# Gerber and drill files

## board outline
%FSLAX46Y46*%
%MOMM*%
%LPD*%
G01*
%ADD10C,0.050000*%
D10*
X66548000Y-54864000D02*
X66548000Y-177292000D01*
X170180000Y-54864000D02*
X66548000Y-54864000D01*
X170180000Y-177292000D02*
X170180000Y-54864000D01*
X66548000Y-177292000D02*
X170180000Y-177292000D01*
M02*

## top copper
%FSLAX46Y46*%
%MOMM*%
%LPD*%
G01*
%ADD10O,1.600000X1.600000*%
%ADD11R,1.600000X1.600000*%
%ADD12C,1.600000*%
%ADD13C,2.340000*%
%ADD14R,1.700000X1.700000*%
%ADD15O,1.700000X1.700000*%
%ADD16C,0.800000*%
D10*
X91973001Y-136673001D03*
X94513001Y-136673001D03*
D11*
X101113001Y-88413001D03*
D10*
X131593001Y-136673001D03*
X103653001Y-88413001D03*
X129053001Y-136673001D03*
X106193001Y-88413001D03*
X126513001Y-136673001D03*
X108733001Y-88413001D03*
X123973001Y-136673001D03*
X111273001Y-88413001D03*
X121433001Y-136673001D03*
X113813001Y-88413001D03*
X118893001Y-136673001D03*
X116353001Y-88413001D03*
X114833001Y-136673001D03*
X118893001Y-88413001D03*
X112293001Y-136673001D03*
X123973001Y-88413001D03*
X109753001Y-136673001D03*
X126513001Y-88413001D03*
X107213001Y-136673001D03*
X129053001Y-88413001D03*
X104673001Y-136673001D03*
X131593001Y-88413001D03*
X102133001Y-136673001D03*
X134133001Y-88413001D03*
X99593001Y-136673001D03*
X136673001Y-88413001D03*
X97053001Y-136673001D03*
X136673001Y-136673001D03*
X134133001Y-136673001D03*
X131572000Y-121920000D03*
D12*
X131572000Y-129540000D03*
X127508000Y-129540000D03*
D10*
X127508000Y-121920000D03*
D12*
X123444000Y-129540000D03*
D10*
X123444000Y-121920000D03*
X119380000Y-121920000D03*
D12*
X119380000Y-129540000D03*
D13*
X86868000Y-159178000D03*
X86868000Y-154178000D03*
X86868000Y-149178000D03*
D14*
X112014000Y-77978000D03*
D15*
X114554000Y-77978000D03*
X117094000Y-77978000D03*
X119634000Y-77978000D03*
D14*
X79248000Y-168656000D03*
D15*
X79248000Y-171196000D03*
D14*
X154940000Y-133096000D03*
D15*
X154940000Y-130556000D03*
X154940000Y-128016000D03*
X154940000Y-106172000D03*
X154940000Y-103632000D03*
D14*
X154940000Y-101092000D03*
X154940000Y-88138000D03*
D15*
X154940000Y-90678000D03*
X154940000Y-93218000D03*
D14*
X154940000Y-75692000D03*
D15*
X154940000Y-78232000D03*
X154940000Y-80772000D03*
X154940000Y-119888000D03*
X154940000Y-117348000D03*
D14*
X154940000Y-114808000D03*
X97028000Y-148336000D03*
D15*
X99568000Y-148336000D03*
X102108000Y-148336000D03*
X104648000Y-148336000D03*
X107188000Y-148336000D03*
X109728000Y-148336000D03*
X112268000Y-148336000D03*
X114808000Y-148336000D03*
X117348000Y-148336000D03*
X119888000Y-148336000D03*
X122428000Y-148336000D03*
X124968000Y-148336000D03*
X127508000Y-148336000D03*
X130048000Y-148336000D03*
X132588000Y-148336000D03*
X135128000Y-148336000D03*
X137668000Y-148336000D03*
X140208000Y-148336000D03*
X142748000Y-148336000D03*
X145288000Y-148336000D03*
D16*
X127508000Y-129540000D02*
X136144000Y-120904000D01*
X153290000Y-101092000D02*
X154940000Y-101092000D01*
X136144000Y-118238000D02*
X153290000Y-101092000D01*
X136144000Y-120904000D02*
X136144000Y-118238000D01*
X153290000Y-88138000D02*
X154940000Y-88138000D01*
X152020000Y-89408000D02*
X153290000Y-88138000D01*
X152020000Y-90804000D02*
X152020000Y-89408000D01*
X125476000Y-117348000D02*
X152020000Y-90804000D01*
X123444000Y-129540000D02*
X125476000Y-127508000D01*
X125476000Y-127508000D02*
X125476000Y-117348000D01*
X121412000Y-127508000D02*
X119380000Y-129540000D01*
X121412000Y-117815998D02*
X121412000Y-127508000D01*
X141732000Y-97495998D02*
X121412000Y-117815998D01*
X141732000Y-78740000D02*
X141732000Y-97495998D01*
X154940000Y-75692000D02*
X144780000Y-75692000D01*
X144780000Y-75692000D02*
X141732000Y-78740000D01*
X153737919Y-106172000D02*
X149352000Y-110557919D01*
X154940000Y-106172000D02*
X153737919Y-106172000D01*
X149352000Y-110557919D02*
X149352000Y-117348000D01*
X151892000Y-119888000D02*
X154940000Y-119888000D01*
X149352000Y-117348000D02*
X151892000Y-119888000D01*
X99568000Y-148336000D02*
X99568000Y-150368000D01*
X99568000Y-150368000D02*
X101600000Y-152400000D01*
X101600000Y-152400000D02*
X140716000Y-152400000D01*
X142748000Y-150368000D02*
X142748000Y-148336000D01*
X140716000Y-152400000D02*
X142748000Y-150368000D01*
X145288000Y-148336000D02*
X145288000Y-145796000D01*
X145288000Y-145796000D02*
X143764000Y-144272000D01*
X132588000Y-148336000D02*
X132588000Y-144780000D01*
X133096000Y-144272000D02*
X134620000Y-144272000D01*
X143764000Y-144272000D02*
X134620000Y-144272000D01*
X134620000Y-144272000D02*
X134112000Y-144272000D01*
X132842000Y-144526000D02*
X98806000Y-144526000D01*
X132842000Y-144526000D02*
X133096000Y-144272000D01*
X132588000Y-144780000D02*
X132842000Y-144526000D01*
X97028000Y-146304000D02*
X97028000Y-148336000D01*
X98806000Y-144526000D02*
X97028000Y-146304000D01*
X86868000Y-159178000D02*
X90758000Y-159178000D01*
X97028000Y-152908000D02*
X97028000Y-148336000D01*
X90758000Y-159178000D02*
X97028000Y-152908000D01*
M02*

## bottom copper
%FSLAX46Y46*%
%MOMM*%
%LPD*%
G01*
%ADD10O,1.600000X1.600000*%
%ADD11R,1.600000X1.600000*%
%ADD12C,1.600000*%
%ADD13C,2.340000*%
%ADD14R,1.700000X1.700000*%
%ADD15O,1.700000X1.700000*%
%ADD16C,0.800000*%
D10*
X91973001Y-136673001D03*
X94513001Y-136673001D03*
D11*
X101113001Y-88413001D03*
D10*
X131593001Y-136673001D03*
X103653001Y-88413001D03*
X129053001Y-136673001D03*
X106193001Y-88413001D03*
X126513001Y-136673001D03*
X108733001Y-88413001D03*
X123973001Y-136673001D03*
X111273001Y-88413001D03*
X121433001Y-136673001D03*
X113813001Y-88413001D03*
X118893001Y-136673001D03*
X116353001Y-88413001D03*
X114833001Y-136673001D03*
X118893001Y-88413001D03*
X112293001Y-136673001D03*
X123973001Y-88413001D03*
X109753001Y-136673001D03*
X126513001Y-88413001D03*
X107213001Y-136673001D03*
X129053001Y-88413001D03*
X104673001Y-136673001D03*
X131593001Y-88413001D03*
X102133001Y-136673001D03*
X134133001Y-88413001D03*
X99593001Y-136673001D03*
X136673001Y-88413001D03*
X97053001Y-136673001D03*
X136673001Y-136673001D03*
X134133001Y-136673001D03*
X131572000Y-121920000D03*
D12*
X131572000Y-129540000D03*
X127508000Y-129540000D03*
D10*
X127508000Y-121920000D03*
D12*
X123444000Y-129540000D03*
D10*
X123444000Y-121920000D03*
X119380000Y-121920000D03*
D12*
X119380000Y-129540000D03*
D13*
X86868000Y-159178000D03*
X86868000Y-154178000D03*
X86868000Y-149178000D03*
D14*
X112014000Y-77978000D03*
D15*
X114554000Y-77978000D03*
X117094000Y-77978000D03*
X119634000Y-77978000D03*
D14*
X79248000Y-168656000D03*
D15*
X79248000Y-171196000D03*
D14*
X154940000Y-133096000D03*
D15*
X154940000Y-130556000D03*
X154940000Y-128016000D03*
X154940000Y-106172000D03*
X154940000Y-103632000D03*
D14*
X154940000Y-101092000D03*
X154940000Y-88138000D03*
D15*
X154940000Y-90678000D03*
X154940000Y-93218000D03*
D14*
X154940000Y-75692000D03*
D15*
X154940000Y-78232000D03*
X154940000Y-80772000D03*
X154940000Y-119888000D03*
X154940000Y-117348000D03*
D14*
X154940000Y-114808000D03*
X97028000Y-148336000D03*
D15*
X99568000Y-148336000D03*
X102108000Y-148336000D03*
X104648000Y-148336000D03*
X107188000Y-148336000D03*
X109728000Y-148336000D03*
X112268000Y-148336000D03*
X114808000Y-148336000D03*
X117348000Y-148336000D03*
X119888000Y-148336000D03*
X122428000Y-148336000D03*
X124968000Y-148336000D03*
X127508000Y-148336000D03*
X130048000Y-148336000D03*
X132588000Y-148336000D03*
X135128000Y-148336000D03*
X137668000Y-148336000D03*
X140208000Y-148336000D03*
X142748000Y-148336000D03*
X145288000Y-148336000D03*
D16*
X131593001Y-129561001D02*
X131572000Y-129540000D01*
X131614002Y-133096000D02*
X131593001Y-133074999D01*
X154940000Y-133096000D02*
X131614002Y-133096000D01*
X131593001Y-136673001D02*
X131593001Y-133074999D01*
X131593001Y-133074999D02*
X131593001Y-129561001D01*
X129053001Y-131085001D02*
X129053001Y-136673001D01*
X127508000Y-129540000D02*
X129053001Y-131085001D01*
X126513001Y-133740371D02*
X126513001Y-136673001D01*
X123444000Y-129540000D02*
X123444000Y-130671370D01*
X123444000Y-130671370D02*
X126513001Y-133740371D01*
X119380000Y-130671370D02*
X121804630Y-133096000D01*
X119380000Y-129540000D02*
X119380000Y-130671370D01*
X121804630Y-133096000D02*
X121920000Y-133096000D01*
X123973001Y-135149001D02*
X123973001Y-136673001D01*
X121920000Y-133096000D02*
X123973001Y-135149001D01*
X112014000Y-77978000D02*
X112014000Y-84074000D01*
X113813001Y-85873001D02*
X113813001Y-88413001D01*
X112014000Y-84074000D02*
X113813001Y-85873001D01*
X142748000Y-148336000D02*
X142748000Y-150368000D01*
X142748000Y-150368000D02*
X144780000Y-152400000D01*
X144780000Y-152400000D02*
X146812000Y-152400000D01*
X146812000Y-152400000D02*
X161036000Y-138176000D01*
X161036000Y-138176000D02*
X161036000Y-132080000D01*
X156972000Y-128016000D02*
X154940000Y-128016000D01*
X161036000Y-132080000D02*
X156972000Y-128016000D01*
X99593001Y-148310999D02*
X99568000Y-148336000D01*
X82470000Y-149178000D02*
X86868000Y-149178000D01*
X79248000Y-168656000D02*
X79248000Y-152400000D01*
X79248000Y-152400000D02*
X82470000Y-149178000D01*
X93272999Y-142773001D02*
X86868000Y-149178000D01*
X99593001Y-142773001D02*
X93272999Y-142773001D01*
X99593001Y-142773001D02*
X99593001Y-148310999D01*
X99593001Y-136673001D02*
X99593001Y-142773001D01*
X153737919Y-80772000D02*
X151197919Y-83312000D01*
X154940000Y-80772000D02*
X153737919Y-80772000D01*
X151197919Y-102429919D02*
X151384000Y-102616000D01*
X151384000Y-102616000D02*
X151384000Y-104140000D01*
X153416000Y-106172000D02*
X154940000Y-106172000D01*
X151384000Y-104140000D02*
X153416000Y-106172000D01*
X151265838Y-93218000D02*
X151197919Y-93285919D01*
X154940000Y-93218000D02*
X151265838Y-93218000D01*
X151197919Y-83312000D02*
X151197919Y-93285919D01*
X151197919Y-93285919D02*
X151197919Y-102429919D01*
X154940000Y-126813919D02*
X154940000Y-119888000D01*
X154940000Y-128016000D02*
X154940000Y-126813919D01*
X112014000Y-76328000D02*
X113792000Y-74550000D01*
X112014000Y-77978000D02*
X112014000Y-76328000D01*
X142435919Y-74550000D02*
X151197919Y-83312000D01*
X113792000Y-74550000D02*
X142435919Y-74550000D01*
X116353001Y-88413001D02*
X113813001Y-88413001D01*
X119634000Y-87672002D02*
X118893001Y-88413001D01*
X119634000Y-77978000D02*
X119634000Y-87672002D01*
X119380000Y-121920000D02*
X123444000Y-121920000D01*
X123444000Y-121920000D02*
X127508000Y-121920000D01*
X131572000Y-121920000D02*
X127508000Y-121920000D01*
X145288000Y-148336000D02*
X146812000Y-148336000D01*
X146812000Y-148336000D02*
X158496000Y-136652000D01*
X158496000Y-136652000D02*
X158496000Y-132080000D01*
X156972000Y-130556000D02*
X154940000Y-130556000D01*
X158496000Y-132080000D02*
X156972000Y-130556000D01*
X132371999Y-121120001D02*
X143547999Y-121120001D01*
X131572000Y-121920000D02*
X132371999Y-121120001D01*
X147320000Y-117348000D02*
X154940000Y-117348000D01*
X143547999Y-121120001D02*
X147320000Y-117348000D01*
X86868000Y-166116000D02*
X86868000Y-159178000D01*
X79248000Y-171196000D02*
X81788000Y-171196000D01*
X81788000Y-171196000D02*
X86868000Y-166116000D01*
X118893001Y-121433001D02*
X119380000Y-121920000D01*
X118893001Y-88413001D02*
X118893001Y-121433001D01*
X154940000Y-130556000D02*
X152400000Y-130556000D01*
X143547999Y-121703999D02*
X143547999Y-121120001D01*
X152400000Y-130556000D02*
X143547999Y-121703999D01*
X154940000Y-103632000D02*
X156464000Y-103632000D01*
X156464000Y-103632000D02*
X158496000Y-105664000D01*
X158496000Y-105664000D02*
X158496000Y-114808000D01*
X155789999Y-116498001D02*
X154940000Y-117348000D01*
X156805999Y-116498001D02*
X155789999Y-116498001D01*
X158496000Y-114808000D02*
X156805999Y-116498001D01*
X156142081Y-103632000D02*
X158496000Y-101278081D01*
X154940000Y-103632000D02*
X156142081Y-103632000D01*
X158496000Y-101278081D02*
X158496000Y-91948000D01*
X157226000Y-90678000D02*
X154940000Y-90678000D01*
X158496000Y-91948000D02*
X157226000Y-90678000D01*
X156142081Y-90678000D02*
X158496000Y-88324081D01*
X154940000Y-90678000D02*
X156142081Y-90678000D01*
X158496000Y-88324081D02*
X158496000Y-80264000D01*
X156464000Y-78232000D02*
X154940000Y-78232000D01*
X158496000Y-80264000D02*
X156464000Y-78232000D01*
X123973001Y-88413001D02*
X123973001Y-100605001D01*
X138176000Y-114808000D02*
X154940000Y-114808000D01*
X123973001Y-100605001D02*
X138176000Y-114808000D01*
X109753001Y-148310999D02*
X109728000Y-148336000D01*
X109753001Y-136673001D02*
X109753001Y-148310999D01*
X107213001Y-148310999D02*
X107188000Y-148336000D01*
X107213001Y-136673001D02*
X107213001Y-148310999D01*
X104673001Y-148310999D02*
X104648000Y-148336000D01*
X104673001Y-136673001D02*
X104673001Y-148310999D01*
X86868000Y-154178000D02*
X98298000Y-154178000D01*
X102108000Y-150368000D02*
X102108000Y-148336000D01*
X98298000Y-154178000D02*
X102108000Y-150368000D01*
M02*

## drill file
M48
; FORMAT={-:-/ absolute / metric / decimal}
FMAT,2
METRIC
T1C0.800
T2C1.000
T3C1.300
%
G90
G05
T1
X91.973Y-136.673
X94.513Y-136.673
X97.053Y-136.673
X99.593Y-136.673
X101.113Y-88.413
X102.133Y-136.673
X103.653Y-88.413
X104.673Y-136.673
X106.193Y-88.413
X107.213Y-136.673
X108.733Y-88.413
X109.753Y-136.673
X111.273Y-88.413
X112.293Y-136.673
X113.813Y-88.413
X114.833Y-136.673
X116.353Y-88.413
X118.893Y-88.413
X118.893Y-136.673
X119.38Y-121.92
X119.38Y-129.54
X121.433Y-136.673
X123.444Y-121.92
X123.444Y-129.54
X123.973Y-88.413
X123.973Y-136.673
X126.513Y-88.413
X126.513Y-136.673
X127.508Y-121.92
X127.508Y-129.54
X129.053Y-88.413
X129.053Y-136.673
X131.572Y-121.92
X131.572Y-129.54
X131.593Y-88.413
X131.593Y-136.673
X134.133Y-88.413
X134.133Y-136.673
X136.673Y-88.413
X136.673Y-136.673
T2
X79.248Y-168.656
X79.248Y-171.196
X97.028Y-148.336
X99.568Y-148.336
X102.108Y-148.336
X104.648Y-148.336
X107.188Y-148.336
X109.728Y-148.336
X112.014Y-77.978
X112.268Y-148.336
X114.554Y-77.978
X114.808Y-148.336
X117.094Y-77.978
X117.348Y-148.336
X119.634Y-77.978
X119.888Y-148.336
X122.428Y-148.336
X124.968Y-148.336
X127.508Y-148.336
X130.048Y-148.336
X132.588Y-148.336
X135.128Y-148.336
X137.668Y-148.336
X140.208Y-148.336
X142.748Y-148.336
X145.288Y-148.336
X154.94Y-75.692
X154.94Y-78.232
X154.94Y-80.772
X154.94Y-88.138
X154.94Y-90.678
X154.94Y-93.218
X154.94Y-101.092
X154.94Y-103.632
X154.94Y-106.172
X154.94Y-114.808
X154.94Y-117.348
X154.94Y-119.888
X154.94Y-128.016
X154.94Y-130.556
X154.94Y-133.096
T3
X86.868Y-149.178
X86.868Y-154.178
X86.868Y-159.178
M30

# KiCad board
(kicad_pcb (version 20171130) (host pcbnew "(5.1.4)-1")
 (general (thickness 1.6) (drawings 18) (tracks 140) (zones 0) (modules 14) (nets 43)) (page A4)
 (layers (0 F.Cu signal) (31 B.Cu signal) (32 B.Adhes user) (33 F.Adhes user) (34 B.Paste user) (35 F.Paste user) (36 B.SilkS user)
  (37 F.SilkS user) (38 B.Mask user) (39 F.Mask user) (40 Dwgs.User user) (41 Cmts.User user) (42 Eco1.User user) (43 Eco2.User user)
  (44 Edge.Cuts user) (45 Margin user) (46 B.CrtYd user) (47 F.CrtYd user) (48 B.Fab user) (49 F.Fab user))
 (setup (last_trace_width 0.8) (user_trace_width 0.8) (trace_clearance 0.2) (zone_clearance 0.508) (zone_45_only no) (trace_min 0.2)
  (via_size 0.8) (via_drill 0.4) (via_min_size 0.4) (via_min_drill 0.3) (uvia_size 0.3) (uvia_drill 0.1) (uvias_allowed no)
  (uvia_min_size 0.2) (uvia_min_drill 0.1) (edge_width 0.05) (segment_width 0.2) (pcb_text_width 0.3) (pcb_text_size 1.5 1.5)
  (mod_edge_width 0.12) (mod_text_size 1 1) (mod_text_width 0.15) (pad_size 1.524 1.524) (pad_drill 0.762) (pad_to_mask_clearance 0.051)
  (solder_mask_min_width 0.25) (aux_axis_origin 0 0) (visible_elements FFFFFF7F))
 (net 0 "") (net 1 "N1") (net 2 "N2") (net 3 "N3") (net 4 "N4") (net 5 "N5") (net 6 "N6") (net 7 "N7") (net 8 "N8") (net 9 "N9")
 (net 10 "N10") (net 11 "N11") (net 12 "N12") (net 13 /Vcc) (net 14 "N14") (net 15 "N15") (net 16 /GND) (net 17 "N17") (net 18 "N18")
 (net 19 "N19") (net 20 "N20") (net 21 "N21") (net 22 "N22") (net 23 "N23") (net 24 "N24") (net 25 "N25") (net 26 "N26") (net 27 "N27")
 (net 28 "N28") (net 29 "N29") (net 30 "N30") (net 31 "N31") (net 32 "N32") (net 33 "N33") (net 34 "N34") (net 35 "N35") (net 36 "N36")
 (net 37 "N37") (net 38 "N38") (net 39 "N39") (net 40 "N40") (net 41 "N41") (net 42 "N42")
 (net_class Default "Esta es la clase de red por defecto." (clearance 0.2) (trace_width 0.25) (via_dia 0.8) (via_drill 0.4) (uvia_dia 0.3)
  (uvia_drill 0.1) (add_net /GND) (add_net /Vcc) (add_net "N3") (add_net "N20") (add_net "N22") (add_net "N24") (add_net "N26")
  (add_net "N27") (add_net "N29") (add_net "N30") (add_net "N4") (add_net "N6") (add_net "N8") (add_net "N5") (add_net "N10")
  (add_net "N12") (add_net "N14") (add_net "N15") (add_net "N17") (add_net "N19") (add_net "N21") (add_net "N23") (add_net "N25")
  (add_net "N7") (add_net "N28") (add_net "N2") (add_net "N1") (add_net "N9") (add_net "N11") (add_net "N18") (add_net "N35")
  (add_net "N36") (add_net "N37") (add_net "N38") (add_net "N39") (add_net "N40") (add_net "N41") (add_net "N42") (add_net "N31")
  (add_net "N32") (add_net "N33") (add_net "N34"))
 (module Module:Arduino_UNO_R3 (layer F.Cu) (at 101.113001 88.413001)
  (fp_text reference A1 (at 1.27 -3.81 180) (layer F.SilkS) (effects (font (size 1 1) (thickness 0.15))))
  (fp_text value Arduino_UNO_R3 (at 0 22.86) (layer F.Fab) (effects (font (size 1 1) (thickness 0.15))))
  (pad 32 thru_hole oval (at -9.14 48.26 90) (size 1.6 1.6) (drill 0.8) (layers *.Cu *.Mask) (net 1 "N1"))
  (pad 31 thru_hole oval (at -6.6 48.26 90) (size 1.6 1.6) (drill 0.8) (layers *.Cu *.Mask) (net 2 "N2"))
  (pad 1 thru_hole rect (at 0 0 90) (size 1.6 1.6) (drill 0.8) (layers *.Cu *.Mask) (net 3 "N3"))
  (pad 17 thru_hole oval (at 30.48 48.26 90) (size 1.6 1.6) (drill 0.8) (layers *.Cu *.Mask) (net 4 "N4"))
  (pad 2 thru_hole oval (at 2.54 0 90) (size 1.6 1.6) (drill 0.8) (layers *.Cu *.Mask) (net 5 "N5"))
  (pad 18 thru_hole oval (at 27.94 48.26 90) (size 1.6 1.6) (drill 0.8) (layers *.Cu *.Mask) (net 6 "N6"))
  (pad 3 thru_hole oval (at 5.08 0 90) (size 1.6 1.6) (drill 0.8) (layers *.Cu *.Mask) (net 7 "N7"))
  (pad 19 thru_hole oval (at 25.4 48.26 90) (size 1.6 1.6) (drill 0.8) (layers *.Cu *.Mask) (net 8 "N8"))
  (pad 4 thru_hole oval (at 7.62 0 90) (size 1.6 1.6) (drill 0.8) (layers *.Cu *.Mask) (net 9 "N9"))
  (pad 20 thru_hole oval (at 22.86 48.26 90) (size 1.6 1.6) (drill 0.8) (layers *.Cu *.Mask) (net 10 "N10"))
  (pad 5 thru_hole oval (at 10.16 0 90) (size 1.6 1.6) (drill 0.8) (layers *.Cu *.Mask) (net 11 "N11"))
  (pad 21 thru_hole oval (at 20.32 48.26 90) (size 1.6 1.6) (drill 0.8) (layers *.Cu *.Mask) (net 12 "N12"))
  (pad 6 thru_hole oval (at 12.7 0 90) (size 1.6 1.6) (drill 0.8) (layers *.Cu *.Mask) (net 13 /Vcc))
  (pad 22 thru_hole oval (at 17.78 48.26 90) (size 1.6 1.6) (drill 0.8) (layers *.Cu *.Mask) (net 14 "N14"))
  (pad 7 thru_hole oval (at 15.24 0 90) (size 1.6 1.6) (drill 0.8) (layers *.Cu *.Mask) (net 13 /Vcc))
  (pad 23 thru_hole oval (at 13.72 48.26 90) (size 1.6 1.6) (drill 0.8) (layers *.Cu *.Mask) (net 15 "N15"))
  (pad 8 thru_hole oval (at 17.78 0 90) (size 1.6 1.6) (drill 0.8) (layers *.Cu *.Mask) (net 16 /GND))
  (pad 24 thru_hole oval (at 11.18 48.26 90) (size 1.6 1.6) (drill 0.8) (layers *.Cu *.Mask) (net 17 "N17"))
  (pad 9 thru_hole oval (at 22.86 0 90) (size 1.6 1.6) (drill 0.8) (layers *.Cu *.Mask) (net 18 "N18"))
  (pad 25 thru_hole oval (at 8.64 48.26 90) (size 1.6 1.6) (drill 0.8) (layers *.Cu *.Mask) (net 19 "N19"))
  (pad 10 thru_hole oval (at 25.4 0 90) (size 1.6 1.6) (drill 0.8) (layers *.Cu *.Mask) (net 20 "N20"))
  (pad 26 thru_hole oval (at 6.1 48.26 90) (size 1.6 1.6) (drill 0.8) (layers *.Cu *.Mask) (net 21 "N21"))
  (pad 11 thru_hole oval (at 27.94 0 90) (size 1.6 1.6) (drill 0.8) (layers *.Cu *.Mask) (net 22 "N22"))
  (pad 27 thru_hole oval (at 3.56 48.26 90) (size 1.6 1.6) (drill 0.8) (layers *.Cu *.Mask) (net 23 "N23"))
  (pad 12 thru_hole oval (at 30.48 0 90) (size 1.6 1.6) (drill 0.8) (layers *.Cu *.Mask) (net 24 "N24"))
  (pad 28 thru_hole oval (at 1.02 48.26 90) (size 1.6 1.6) (drill 0.8) (layers *.Cu *.Mask) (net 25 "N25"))
  (pad 13 thru_hole oval (at 33.02 0 90) (size 1.6 1.6) (drill 0.8) (layers *.Cu *.Mask) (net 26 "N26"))
  (pad 29 thru_hole oval (at -1.52 48.26 90) (size 1.6 1.6) (drill 0.8) (layers *.Cu *.Mask) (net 13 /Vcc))
  (pad 14 thru_hole oval (at 35.56 0 90) (size 1.6 1.6) (drill 0.8) (layers *.Cu *.Mask) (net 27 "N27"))
  (pad 30 thru_hole oval (at -4.06 48.26 90) (size 1.6 1.6) (drill 0.8) (layers *.Cu *.Mask) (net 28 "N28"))
  (pad 15 thru_hole oval (at 35.56 48.26 90) (size 1.6 1.6) (drill 0.8) (layers *.Cu *.Mask) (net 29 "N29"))
  (pad 16 thru_hole oval (at 33.02 48.26 90) (size 1.6 1.6) (drill 0.8) (layers *.Cu *.Mask) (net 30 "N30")))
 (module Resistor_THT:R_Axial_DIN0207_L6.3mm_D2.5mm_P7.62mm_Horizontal (layer F.Cu) (at 131.572 129.54 90)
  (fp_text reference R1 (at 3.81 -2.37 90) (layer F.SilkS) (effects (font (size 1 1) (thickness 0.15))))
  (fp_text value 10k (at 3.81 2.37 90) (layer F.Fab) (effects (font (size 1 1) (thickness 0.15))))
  (pad 2 thru_hole oval (at 7.62 0 90) (size 1.6 1.6) (drill 0.8) (layers *.Cu *.Mask) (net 16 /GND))
  (pad 1 thru_hole circle (at 0 0 90) (size 1.6 1.6) (drill 0.8) (layers *.Cu *.Mask) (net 4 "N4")))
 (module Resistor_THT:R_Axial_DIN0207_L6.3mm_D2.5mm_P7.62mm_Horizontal (layer F.Cu) (at 127.508 129.54 90)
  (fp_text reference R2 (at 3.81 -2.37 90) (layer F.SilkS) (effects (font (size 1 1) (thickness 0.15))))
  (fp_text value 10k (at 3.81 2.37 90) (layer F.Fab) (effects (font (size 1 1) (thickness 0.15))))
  (pad 1 thru_hole circle (at 0 0 90) (size 1.6 1.6) (drill 0.8) (layers *.Cu *.Mask) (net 6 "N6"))
  (pad 2 thru_hole oval (at 7.62 0 90) (size 1.6 1.6) (drill 0.8) (layers *.Cu *.Mask) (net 16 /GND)))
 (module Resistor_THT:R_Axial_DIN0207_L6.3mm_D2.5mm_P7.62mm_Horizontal (layer F.Cu) (at 123.444 129.54 90)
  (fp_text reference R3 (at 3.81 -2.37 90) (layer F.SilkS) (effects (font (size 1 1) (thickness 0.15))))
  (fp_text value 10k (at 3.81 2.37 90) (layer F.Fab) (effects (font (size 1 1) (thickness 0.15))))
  (pad 1 thru_hole circle (at 0 0 90) (size 1.6 1.6) (drill 0.8) (layers *.Cu *.Mask) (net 8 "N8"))
  (pad 2 thru_hole oval (at 7.62 0 90) (size 1.6 1.6) (drill 0.8) (layers *.Cu *.Mask) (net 16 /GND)))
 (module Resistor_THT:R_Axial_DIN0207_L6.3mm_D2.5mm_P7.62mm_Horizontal (layer F.Cu) (at 119.38 129.54 90)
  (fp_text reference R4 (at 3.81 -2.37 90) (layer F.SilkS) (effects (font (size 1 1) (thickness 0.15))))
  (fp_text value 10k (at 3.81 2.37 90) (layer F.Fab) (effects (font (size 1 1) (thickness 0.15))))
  (pad 2 thru_hole oval (at 7.62 0 90) (size 1.6 1.6) (drill 0.8) (layers *.Cu *.Mask) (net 16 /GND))
  (pad 1 thru_hole circle (at 0 0 90) (size 1.6 1.6) (drill 0.8) (layers *.Cu *.Mask) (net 10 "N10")))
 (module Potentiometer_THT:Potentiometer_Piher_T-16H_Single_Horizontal (layer F.Cu) (at 86.868 149.178 180)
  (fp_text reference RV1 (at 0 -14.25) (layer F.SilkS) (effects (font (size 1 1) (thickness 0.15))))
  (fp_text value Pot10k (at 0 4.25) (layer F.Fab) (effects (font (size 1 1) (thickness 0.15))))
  (pad 3 thru_hole circle (at 0 -10 180) (size 2.34 2.34) (drill 1.3) (layers *.Cu *.Mask) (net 16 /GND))
  (pad 2 thru_hole circle (at 0 -5 180) (size 2.34 2.34) (drill 1.3) (layers *.Cu *.Mask) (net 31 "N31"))
  (pad 1 thru_hole circle (at 0 0 180) (size 2.34 2.34) (drill 1.3) (layers *.Cu *.Mask) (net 13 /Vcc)))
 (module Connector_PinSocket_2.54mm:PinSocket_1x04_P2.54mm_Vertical (layer F.Cu) (at 112.014 77.978 90)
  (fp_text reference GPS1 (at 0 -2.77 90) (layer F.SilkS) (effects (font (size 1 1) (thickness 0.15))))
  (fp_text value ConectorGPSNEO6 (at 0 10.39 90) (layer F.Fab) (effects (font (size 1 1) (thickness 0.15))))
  (pad 1 thru_hole rect (at 0 0 90) (size 1.7 1.7) (drill 1) (layers *.Cu *.Mask) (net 13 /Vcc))
  (pad 2 thru_hole oval (at 0 2.54 90) (size 1.7 1.7) (drill 1) (layers *.Cu *.Mask))
  (pad 3 thru_hole oval (at 0 5.08 90) (size 1.7 1.7) (drill 1) (layers *.Cu *.Mask))
  (pad 4 thru_hole oval (at 0 7.62 90) (size 1.7 1.7) (drill 1) (layers *.Cu *.Mask) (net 16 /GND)))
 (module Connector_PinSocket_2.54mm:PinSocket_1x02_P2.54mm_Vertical (layer F.Cu) (at 79.248 168.656)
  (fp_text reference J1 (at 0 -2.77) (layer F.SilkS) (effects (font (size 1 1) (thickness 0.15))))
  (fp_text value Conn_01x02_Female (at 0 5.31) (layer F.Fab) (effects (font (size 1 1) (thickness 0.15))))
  (pad 1 thru_hole rect (at 0 0) (size 1.7 1.7) (drill 1) (layers *.Cu *.Mask) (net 13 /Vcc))
  (pad 2 thru_hole oval (at 0 2.54) (size 1.7 1.7) (drill 1) (layers *.Cu *.Mask) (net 16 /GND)))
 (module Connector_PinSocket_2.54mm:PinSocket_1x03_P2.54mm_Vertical (layer F.Cu) (at 154.94 133.096 180)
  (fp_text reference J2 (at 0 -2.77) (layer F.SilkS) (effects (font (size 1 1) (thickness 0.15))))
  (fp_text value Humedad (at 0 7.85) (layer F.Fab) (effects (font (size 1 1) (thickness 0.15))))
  (pad 1 thru_hole rect (at 0 0 180) (size 1.7 1.7) (drill 1) (layers *.Cu *.Mask) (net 4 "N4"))
  (pad 2 thru_hole oval (at 0 2.54 180) (size 1.7 1.7) (drill 1) (layers *.Cu *.Mask) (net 16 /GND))
  (pad 3 thru_hole oval (at 0 5.08 180) (size 1.7 1.7) (drill 1) (layers *.Cu *.Mask) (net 13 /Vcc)))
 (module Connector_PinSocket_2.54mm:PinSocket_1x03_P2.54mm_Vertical (layer F.Cu) (at 154.94 101.092)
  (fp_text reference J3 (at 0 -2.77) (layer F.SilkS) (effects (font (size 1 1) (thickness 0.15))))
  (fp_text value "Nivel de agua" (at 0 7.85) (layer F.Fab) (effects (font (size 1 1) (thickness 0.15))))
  (pad 3 thru_hole oval (at 0 5.08) (size 1.7 1.7) (drill 1) (layers *.Cu *.Mask) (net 13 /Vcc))
  (pad 2 thru_hole oval (at 0 2.54) (size 1.7 1.7) (drill 1) (layers *.Cu *.Mask) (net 16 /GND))
  (pad 1 thru_hole rect (at 0 0) (size 1.7 1.7) (drill 1) (layers *.Cu *.Mask) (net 6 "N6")))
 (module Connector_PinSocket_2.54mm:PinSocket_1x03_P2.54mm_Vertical (layer F.Cu) (at 154.94 88.138)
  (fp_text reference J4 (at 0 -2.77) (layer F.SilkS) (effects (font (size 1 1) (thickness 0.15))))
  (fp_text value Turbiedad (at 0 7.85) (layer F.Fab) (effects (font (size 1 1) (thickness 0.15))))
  (pad 1 thru_hole rect (at 0 0) (size 1.7 1.7) (drill 1) (layers *.Cu *.Mask) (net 8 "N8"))
  (pad 2 thru_hole oval (at 0 2.54) (size 1.7 1.7) (drill 1) (layers *.Cu *.Mask) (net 16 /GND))
  (pad 3 thru_hole oval (at 0 5.08) (size 1.7 1.7) (drill 1) (layers *.Cu *.Mask) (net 13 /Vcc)))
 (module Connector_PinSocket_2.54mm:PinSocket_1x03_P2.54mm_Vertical (layer F.Cu) (at 154.94 75.692)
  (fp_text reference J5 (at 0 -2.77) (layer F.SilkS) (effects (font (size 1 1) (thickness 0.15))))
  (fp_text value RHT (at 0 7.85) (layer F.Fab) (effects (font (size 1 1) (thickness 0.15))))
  (pad 1 thru_hole rect (at 0 0) (size 1.7 1.7) (drill 1) (layers *.Cu *.Mask) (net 10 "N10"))
  (pad 2 thru_hole oval (at 0 2.54) (size 1.7 1.7) (drill 1) (layers *.Cu *.Mask) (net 16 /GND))
  (pad 3 thru_hole oval (at 0 5.08) (size 1.7 1.7) (drill 1) (layers *.Cu *.Mask) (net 13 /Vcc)))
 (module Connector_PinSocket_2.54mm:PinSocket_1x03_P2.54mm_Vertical (layer F.Cu) (at 154.94 114.808)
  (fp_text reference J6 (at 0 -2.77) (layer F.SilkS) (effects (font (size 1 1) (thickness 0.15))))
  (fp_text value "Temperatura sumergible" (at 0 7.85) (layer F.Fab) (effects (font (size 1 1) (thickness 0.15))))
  (pad 3 thru_hole oval (at 0 5.08) (size 1.7 1.7) (drill 1) (layers *.Cu *.Mask) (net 13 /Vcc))
  (pad 2 thru_hole oval (at 0 2.54) (size 1.7 1.7) (drill 1) (layers *.Cu *.Mask) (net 16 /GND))
  (pad 1 thru_hole rect (at 0 0) (size 1.7 1.7) (drill 1) (layers *.Cu *.Mask) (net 18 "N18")))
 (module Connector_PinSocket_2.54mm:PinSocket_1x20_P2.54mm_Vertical (layer F.Cu) (at 97.028 148.336 90)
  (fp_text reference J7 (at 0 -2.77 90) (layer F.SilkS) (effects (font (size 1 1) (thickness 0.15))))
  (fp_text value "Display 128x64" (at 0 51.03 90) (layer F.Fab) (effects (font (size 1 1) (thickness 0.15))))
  (pad 1 thru_hole rect (at 0 0 90) (size 1.7 1.7) (drill 1) (layers *.Cu *.Mask) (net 16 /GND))
  (pad 2 thru_hole oval (at 0 2.54 90) (size 1.7 1.7) (drill 1) (layers *.Cu *.Mask) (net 13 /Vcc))
  (pad 3 thru_hole oval (at 0 5.08 90) (size 1.7 1.7) (drill 1) (layers *.Cu *.Mask) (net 31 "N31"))
  (pad 4 thru_hole oval (at 0 7.62 90) (size 1.7 1.7) (drill 1) (layers *.Cu *.Mask) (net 23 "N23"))
  (pad 5 thru_hole oval (at 0 10.16 90) (size 1.7 1.7) (drill 1) (layers *.Cu *.Mask) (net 21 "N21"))
  (pad 6 thru_hole oval (at 0 12.7 90) (size 1.7 1.7) (drill 1) (layers *.Cu *.Mask) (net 19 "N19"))
  (pad 7 thru_hole oval (at 0 15.24 90) (size 1.7 1.7) (drill 1) (layers *.Cu *.Mask) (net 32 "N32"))
  (pad 8 thru_hole oval (at 0 17.78 90) (size 1.7 1.7) (drill 1) (layers *.Cu *.Mask) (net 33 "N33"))
  (pad 9 thru_hole oval (at 0 20.32 90) (size 1.7 1.7) (drill 1) (layers *.Cu *.Mask) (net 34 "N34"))
  (pad 10 thru_hole oval (at 0 22.86 90) (size 1.7 1.7) (drill 1) (layers *.Cu *.Mask) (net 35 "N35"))
  (pad 11 thru_hole oval (at 0 25.4 90) (size 1.7 1.7) (drill 1) (layers *.Cu *.Mask) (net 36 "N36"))
  (pad 12 thru_hole oval (at 0 27.94 90) (size 1.7 1.7) (drill 1) (layers *.Cu *.Mask) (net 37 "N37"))
  (pad 13 thru_hole oval (at 0 30.48 90) (size 1.7 1.7) (drill 1) (layers *.Cu *.Mask) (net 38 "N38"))
  (pad 14 thru_hole oval (at 0 33.02 90) (size 1.7 1.7) (drill 1) (layers *.Cu *.Mask) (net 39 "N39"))
  (pad 15 thru_hole oval (at 0 35.56 90) (size 1.7 1.7) (drill 1) (layers *.Cu *.Mask) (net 16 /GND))
  (pad 16 thru_hole oval (at 0 38.1 90) (size 1.7 1.7) (drill 1) (layers *.Cu *.Mask) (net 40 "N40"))
  (pad 17 thru_hole oval (at 0 40.64 90) (size 1.7 1.7) (drill 1) (layers *.Cu *.Mask) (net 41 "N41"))
  (pad 18 thru_hole oval (at 0 43.18 90) (size 1.7 1.7) (drill 1) (layers *.Cu *.Mask) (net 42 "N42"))
  (pad 19 thru_hole oval (at 0 45.72 90) (size 1.7 1.7) (drill 1) (layers *.Cu *.Mask) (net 13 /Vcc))
  (pad 20 thru_hole oval (at 0 48.26 90) (size 1.7 1.7) (drill 1) (layers *.Cu *.Mask) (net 16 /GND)))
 (gr_line (start 66.548 54.864) (end 66.548 177.292) (layer Edge.Cuts) (width 0.05))
 (gr_line (start 170.18 54.864) (end 66.548 54.864) (layer Edge.Cuts) (width 0.05))
 (gr_line (start 170.18 177.292) (end 170.18 54.864) (layer Edge.Cuts) (width 0.05))
 (gr_line (start 66.548 177.292) (end 170.18 177.292) (layer Edge.Cuts) (width 0.05))
 (segment (start 131.593001 129.561001) (end 131.572 129.54) (width 0.8) (layer B.Cu) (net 4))
 (segment (start 131.614002 133.096) (end 131.593001 133.074999) (width 0.8) (layer B.Cu) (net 4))
 (segment (start 154.94 133.096) (end 131.614002 133.096) (width 0.8) (layer B.Cu) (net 4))
 (segment (start 131.593001 136.673001) (end 131.593001 133.074999) (width 0.8) (layer B.Cu) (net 4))
 (segment (start 131.593001 133.074999) (end 131.593001 129.561001) (width 0.8) (layer B.Cu) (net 4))
 (segment (start 129.053001 131.085001) (end 129.053001 136.673001) (width 0.8) (layer B.Cu) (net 6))
 (segment (start 127.508 129.54) (end 129.053001 131.085001) (width 0.8) (layer B.Cu) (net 6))
 (segment (start 127.508 129.54) (end 136.144 120.904) (width 0.8) (layer F.Cu) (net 6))
 (segment (start 153.29 101.092) (end 154.94 101.092) (width 0.8) (layer F.Cu) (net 6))
 (segment (start 136.144 118.238) (end 153.29 101.092) (width 0.8) (layer F.Cu) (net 6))
 (segment (start 136.144 120.904) (end 136.144 118.238) (width 0.8) (layer F.Cu) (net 6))
 (segment (start 126.513001 133.740371) (end 126.513001 136.673001) (width 0.8) (layer B.Cu) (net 8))
 (segment (start 123.444 129.54) (end 123.444 130.67137) (width 0.8) (layer B.Cu) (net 8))
 (segment (start 123.444 130.67137) (end 126.513001 133.740371) (width 0.8) (layer B.Cu) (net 8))
 (segment (start 153.29 88.138) (end 154.94 88.138) (width 0.8) (layer F.Cu) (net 8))
 (segment (start 152.02 89.408) (end 153.29 88.138) (width 0.8) (layer F.Cu) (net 8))
 (segment (start 152.02 90.804) (end 152.02 89.408) (width 0.8) (layer F.Cu) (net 8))
 (segment (start 125.476 117.348) (end 152.02 90.804) (width 0.8) (layer F.Cu) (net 8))
 (segment (start 123.444 129.54) (end 125.476 127.508) (width 0.8) (layer F.Cu) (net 8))
 (segment (start 125.476 127.508) (end 125.476 117.348) (width 0.8) (layer F.Cu) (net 8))
 (segment (start 119.38 130.67137) (end 121.80463 133.096) (width 0.8) (layer B.Cu) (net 10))
 (segment (start 119.38 129.54) (end 119.38 130.67137) (width 0.8) (layer B.Cu) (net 10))
 (segment (start 121.80463 133.096) (end 121.92 133.096) (width 0.8) (layer B.Cu) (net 10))
 (segment (start 123.973001 135.149001) (end 123.973001 136.673001) (width 0.8) (layer B.Cu) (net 10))
 (segment (start 121.92 133.096) (end 123.973001 135.149001) (width 0.8) (layer B.Cu) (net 10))
 (segment (start 121.412 127.508) (end 119.38 129.54) (width 0.8) (layer F.Cu) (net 10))
 (segment (start 121.412 117.815998) (end 121.412 127.508) (width 0.8) (layer F.Cu) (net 10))
 (segment (start 141.732 97.495998) (end 121.412 117.815998) (width 0.8) (layer F.Cu) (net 10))
 (segment (start 141.732 78.74) (end 141.732 97.495998) (width 0.8) (layer F.Cu) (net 10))
 (segment (start 154.94 75.692) (end 144.78 75.692) (width 0.8) (layer F.Cu) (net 10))
 (segment (start 144.78 75.692) (end 141.732 78.74) (width 0.8) (layer F.Cu) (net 10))
 (segment (start 112.014 77.978) (end 112.014 84.074) (width 0.8) (layer B.Cu) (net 13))
 (segment (start 113.813001 85.873001) (end 113.813001 88.413001) (width 0.8) (layer B.Cu) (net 13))
 (segment (start 112.014 84.074) (end 113.813001 85.873001) (width 0.8) (layer B.Cu) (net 13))
 (segment (start 142.748 148.336) (end 142.748 150.368) (width 0.8) (layer B.Cu) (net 13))
 (segment (start 142.748 150.368) (end 144.78 152.4) (width 0.8) (layer B.Cu) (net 13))
 (segment (start 144.78 152.4) (end 146.812 152.4) (width 0.8) (layer B.Cu) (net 13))
 (segment (start 146.812 152.4) (end 161.036 138.176) (width 0.8) (layer B.Cu) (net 13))
 (segment (start 161.036 138.176) (end 161.036 132.08) (width 0.8) (layer B.Cu) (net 13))
 (segment (start 156.972 128.016) (end 154.94 128.016) (width 0.8) (layer B.Cu) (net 13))
 (segment (start 161.036 132.08) (end 156.972 128.016) (width 0.8) (layer B.Cu) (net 13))
 (segment (start 99.593001 148.310999) (end 99.568 148.336) (width 0.8) (layer B.Cu) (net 13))
 (segment (start 82.47 149.178) (end 86.868 149.178) (width 0.8) (layer B.Cu) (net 13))
 (segment (start 79.248 168.656) (end 79.248 152.4) (width 0.8) (layer B.Cu) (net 13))
 (segment (start 79.248 152.4) (end 82.47 149.178) (width 0.8) (layer B.Cu) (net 13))
 (segment (start 93.272999 142.773001) (end 86.868 149.178) (width 0.8) (layer B.Cu) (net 13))
 (segment (start 99.593001 142.773001) (end 93.272999 142.773001) (width 0.8) (layer B.Cu) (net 13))
 (segment (start 99.593001 142.773001) (end 99.593001 148.310999) (width 0.8) (layer B.Cu) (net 13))
 (segment (start 99.593001 136.673001) (end 99.593001 142.773001) (width 0.8) (layer B.Cu) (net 13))
 (segment (start 153.737919 80.772) (end 151.197919 83.312) (width 0.8) (layer B.Cu) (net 13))
 (segment (start 154.94 80.772) (end 153.737919 80.772) (width 0.8) (layer B.Cu) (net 13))
 (segment (start 151.197919 102.429919) (end 151.384 102.616) (width 0.8) (layer B.Cu) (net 13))
 (segment (start 151.384 102.616) (end 151.384 104.14) (width 0.8) (layer B.Cu) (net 13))
 (segment (start 153.416 106.172) (end 154.94 106.172) (width 0.8) (layer B.Cu) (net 13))
 (segment (start 151.384 104.14) (end 153.416 106.172) (width 0.8) (layer B.Cu) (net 13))
 (segment (start 151.265838 93.218) (end 151.197919 93.285919) (width 0.8) (layer B.Cu) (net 13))
 (segment (start 154.94 93.218) (end 151.265838 93.218) (width 0.8) (layer B.Cu) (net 13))
 (segment (start 151.197919 83.312) (end 151.197919 93.285919) (width 0.8) (layer B.Cu) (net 13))
 (segment (start 151.197919 93.285919) (end 151.197919 102.429919) (width 0.8) (layer B.Cu) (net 13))
 (segment (start 153.737919 106.172) (end 149.352 110.557919) (width 0.8) (layer F.Cu) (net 13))
 (segment (start 154.94 106.172) (end 153.737919 106.172) (width 0.8) (layer F.Cu) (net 13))
 (segment (start 149.352 110.557919) (end 149.352 117.348) (width 0.8) (layer F.Cu) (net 13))
 (segment (start 151.892 119.888) (end 154.94 119.888) (width 0.8) (layer F.Cu) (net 13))
 (segment (start 149.352 117.348) (end 151.892 119.888) (width 0.8) (layer F.Cu) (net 13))
 (segment (start 154.94 126.813919) (end 154.94 119.888) (width 0.8) (layer B.Cu) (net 13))
 (segment (start 154.94 128.016) (end 154.94 126.813919) (width 0.8) (layer B.Cu) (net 13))
 (segment (start 112.014 76.328) (end 113.792 74.55) (width 0.8) (layer B.Cu) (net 13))
 (segment (start 112.014 77.978) (end 112.014 76.328) (width 0.8) (layer B.Cu) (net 13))
 (segment (start 142.435919 74.55) (end 151.197919 83.312) (width 0.8) (layer B.Cu) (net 13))
 (segment (start 113.792 74.55) (end 142.435919 74.55) (width 0.8) (layer B.Cu) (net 13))
 (segment (start 116.353001 88.413001) (end 113.813001 88.413001) (width 0.8) (layer B.Cu) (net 13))
 (segment (start 99.568 148.336) (end 99.568 150.368) (width 0.8) (layer F.Cu) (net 13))
 (segment (start 99.568 150.368) (end 101.6 152.4) (width 0.8) (layer F.Cu) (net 13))
 (segment (start 101.6 152.4) (end 140.716 152.4) (width 0.8) (layer F.Cu) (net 13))
 (segment (start 142.748 150.368) (end 142.748 148.336) (width 0.8) (layer F.Cu) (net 13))
 (segment (start 140.716 152.4) (end 142.748 150.368) (width 0.8) (layer F.Cu) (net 13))
 (segment (start 119.634 87.672002) (end 118.893001 88.413001) (width 0.8) (layer B.Cu) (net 16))
 (segment (start 119.634 77.978) (end 119.634 87.672002) (width 0.8) (layer B.Cu) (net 16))
 (segment (start 119.38 121.92) (end 123.444 121.92) (width 0.8) (layer B.Cu) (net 16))
 (segment (start 123.444 121.92) (end 127.508 121.92) (width 0.8) (layer B.Cu) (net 16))
 (segment (start 131.572 121.92) (end 127.508 121.92) (width 0.8) (layer B.Cu) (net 16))
 (segment (start 145.288 148.336) (end 146.812 148.336) (width 0.8) (layer B.Cu) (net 16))
 (segment (start 146.812 148.336) (end 158.496 136.652) (width 0.8) (layer B.Cu) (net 16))
 (segment (start 158.496 136.652) (end 158.496 132.08) (width 0.8) (layer B.Cu) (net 16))
 (segment (start 156.972 130.556) (end 154.94 130.556) (width 0.8) (layer B.Cu) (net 16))
 (segment (start 158.496 132.08) (end 156.972 130.556) (width 0.8) (layer B.Cu) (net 16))
 (segment (start 132.371999 121.120001) (end 143.547999 121.120001) (width 0.8) (layer B.Cu) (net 16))
 (segment (start 131.572 121.92) (end 132.371999 121.120001) (width 0.8) (layer B.Cu) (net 16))
 (segment (start 147.32 117.348) (end 154.94 117.348) (width 0.8) (layer B.Cu) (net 16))
 (segment (start 143.547999 121.120001) (end 147.32 117.348) (width 0.8) (layer B.Cu) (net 16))
 (segment (start 86.868 166.116) (end 86.868 159.178) (width 0.8) (layer B.Cu) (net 16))
 (segment (start 79.248 171.196) (end 81.788 171.196) (width 0.8) (layer B.Cu) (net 16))
 (segment (start 81.788 171.196) (end 86.868 166.116) (width 0.8) (layer B.Cu) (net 16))
 (segment (start 145.288 148.336) (end 145.288 145.796) (width 0.8) (layer F.Cu) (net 16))
 (segment (start 145.288 145.796) (end 143.764 144.272) (width 0.8) (layer F.Cu) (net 16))
 (segment (start 132.588 148.336) (end 132.588 144.78) (width 0.8) (layer F.Cu) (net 16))
 (segment (start 133.096 144.272) (end 134.62 144.272) (width 0.8) (layer F.Cu) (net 16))
 (segment (start 143.764 144.272) (end 134.62 144.272) (width 0.8) (layer F.Cu) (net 16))
 (segment (start 134.62 144.272) (end 134.112 144.272) (width 0.8) (layer F.Cu) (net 16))
 (segment (start 132.842 144.526) (end 98.806 144.526) (width 0.8) (layer F.Cu) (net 16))
 (segment (start 132.842 144.526) (end 133.096 144.272) (width 0.8) (layer F.Cu) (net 16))
 (segment (start 132.588 144.78) (end 132.842 144.526) (width 0.8) (layer F.Cu) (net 16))
 (segment (start 97.028 146.304) (end 97.028 148.336) (width 0.8) (layer F.Cu) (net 16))
 (segment (start 98.806 144.526) (end 97.028 146.304) (width 0.8) (layer F.Cu) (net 16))
 (segment (start 86.868 159.178) (end 90.758 159.178) (width 0.8) (layer F.Cu) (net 16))
 (segment (start 97.028 152.908) (end 97.028 148.336) (width 0.8) (layer F.Cu) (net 16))
 (segment (start 90.758 159.178) (end 97.028 152.908) (width 0.8) (layer F.Cu) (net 16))
 (segment (start 118.893001 121.433001) (end 119.38 121.92) (width 0.8) (layer B.Cu) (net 16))
 (segment (start 118.893001 88.413001) (end 118.893001 121.433001) (width 0.8) (layer B.Cu) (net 16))
 (segment (start 154.94 130.556) (end 152.4 130.556) (width 0.8) (layer B.Cu) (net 16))
 (segment (start 143.547999 121.703999) (end 143.547999 121.120001) (width 0.8) (layer B.Cu) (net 16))
 (segment (start 152.4 130.556) (end 143.547999 121.703999) (width 0.8) (layer B.Cu) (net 16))
 (segment (start 154.94 103.632) (end 156.464 103.632) (width 0.8) (layer B.Cu) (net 16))
 (segment (start 156.464 103.632) (end 158.496 105.664) (width 0.8) (layer B.Cu) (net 16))
 (segment (start 158.496 105.664) (end 158.496 114.808) (width 0.8) (layer B.Cu) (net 16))
 (segment (start 155.789999 116.498001) (end 154.94 117.348) (width 0.8) (layer B.Cu) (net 16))
 (segment (start 156.805999 116.498001) (end 155.789999 116.498001) (width 0.8) (layer B.Cu) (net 16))
 (segment (start 158.496 114.808) (end 156.805999 116.498001) (width 0.8) (layer B.Cu) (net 16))
 (segment (start 156.142081 103.632) (end 158.496 101.278081) (width 0.8) (layer B.Cu) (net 16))
 (segment (start 154.94 103.632) (end 156.142081 103.632) (width 0.8) (layer B.Cu) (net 16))
 (segment (start 158.496 101.278081) (end 158.496 91.948) (width 0.8) (layer B.Cu) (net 16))
 (segment (start 157.226 90.678) (end 154.94 90.678) (width 0.8) (layer B.Cu) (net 16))
 (segment (start 158.496 91.948) (end 157.226 90.678) (width 0.8) (layer B.Cu) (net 16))
 (segment (start 156.142081 90.678) (end 158.496 88.324081) (width 0.8) (layer B.Cu) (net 16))
 (segment (start 154.94 90.678) (end 156.142081 90.678) (width 0.8) (layer B.Cu) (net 16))
 (segment (start 158.496 88.324081) (end 158.496 80.264) (width 0.8) (layer B.Cu) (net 16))
 (segment (start 156.464 78.232) (end 154.94 78.232) (width 0.8) (layer B.Cu) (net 16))
 (segment (start 158.496 80.264) (end 156.464 78.232) (width 0.8) (layer B.Cu) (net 16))
 (segment (start 123.973001 88.413001) (end 123.973001 100.605001) (width 0.8) (layer B.Cu) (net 18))
 (segment (start 138.176 114.808) (end 154.94 114.808) (width 0.8) (layer B.Cu) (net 18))
 (segment (start 123.973001 100.605001) (end 138.176 114.808) (width 0.8) (layer B.Cu) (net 18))
 (segment (start 109.753001 148.310999) (end 109.728 148.336) (width 0.8) (layer B.Cu) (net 19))
 (segment (start 109.753001 136.673001) (end 109.753001 148.310999) (width 0.8) (layer B.Cu) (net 19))
 (segment (start 107.213001 148.310999) (end 107.188 148.336) (width 0.8) (layer B.Cu) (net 21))
 (segment (start 107.213001 136.673001) (end 107.213001 148.310999) (width 0.8) (layer B.Cu) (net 21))
 (segment (start 104.673001 148.310999) (end 104.648 148.336) (width 0.8) (layer B.Cu) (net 23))
 (segment (start 104.673001 136.673001) (end 104.673001 148.310999) (width 0.8) (layer B.Cu) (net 23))
 (segment (start 86.868 154.178) (end 98.298 154.178) (width 0.8) (layer B.Cu) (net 31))
 (segment (start 102.108 150.368) (end 102.108 148.336) (width 0.8) (layer B.Cu) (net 31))
 (segment (start 98.298 154.178) (end 102.108 150.368) (width 0.8) (layer B.Cu) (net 31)))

